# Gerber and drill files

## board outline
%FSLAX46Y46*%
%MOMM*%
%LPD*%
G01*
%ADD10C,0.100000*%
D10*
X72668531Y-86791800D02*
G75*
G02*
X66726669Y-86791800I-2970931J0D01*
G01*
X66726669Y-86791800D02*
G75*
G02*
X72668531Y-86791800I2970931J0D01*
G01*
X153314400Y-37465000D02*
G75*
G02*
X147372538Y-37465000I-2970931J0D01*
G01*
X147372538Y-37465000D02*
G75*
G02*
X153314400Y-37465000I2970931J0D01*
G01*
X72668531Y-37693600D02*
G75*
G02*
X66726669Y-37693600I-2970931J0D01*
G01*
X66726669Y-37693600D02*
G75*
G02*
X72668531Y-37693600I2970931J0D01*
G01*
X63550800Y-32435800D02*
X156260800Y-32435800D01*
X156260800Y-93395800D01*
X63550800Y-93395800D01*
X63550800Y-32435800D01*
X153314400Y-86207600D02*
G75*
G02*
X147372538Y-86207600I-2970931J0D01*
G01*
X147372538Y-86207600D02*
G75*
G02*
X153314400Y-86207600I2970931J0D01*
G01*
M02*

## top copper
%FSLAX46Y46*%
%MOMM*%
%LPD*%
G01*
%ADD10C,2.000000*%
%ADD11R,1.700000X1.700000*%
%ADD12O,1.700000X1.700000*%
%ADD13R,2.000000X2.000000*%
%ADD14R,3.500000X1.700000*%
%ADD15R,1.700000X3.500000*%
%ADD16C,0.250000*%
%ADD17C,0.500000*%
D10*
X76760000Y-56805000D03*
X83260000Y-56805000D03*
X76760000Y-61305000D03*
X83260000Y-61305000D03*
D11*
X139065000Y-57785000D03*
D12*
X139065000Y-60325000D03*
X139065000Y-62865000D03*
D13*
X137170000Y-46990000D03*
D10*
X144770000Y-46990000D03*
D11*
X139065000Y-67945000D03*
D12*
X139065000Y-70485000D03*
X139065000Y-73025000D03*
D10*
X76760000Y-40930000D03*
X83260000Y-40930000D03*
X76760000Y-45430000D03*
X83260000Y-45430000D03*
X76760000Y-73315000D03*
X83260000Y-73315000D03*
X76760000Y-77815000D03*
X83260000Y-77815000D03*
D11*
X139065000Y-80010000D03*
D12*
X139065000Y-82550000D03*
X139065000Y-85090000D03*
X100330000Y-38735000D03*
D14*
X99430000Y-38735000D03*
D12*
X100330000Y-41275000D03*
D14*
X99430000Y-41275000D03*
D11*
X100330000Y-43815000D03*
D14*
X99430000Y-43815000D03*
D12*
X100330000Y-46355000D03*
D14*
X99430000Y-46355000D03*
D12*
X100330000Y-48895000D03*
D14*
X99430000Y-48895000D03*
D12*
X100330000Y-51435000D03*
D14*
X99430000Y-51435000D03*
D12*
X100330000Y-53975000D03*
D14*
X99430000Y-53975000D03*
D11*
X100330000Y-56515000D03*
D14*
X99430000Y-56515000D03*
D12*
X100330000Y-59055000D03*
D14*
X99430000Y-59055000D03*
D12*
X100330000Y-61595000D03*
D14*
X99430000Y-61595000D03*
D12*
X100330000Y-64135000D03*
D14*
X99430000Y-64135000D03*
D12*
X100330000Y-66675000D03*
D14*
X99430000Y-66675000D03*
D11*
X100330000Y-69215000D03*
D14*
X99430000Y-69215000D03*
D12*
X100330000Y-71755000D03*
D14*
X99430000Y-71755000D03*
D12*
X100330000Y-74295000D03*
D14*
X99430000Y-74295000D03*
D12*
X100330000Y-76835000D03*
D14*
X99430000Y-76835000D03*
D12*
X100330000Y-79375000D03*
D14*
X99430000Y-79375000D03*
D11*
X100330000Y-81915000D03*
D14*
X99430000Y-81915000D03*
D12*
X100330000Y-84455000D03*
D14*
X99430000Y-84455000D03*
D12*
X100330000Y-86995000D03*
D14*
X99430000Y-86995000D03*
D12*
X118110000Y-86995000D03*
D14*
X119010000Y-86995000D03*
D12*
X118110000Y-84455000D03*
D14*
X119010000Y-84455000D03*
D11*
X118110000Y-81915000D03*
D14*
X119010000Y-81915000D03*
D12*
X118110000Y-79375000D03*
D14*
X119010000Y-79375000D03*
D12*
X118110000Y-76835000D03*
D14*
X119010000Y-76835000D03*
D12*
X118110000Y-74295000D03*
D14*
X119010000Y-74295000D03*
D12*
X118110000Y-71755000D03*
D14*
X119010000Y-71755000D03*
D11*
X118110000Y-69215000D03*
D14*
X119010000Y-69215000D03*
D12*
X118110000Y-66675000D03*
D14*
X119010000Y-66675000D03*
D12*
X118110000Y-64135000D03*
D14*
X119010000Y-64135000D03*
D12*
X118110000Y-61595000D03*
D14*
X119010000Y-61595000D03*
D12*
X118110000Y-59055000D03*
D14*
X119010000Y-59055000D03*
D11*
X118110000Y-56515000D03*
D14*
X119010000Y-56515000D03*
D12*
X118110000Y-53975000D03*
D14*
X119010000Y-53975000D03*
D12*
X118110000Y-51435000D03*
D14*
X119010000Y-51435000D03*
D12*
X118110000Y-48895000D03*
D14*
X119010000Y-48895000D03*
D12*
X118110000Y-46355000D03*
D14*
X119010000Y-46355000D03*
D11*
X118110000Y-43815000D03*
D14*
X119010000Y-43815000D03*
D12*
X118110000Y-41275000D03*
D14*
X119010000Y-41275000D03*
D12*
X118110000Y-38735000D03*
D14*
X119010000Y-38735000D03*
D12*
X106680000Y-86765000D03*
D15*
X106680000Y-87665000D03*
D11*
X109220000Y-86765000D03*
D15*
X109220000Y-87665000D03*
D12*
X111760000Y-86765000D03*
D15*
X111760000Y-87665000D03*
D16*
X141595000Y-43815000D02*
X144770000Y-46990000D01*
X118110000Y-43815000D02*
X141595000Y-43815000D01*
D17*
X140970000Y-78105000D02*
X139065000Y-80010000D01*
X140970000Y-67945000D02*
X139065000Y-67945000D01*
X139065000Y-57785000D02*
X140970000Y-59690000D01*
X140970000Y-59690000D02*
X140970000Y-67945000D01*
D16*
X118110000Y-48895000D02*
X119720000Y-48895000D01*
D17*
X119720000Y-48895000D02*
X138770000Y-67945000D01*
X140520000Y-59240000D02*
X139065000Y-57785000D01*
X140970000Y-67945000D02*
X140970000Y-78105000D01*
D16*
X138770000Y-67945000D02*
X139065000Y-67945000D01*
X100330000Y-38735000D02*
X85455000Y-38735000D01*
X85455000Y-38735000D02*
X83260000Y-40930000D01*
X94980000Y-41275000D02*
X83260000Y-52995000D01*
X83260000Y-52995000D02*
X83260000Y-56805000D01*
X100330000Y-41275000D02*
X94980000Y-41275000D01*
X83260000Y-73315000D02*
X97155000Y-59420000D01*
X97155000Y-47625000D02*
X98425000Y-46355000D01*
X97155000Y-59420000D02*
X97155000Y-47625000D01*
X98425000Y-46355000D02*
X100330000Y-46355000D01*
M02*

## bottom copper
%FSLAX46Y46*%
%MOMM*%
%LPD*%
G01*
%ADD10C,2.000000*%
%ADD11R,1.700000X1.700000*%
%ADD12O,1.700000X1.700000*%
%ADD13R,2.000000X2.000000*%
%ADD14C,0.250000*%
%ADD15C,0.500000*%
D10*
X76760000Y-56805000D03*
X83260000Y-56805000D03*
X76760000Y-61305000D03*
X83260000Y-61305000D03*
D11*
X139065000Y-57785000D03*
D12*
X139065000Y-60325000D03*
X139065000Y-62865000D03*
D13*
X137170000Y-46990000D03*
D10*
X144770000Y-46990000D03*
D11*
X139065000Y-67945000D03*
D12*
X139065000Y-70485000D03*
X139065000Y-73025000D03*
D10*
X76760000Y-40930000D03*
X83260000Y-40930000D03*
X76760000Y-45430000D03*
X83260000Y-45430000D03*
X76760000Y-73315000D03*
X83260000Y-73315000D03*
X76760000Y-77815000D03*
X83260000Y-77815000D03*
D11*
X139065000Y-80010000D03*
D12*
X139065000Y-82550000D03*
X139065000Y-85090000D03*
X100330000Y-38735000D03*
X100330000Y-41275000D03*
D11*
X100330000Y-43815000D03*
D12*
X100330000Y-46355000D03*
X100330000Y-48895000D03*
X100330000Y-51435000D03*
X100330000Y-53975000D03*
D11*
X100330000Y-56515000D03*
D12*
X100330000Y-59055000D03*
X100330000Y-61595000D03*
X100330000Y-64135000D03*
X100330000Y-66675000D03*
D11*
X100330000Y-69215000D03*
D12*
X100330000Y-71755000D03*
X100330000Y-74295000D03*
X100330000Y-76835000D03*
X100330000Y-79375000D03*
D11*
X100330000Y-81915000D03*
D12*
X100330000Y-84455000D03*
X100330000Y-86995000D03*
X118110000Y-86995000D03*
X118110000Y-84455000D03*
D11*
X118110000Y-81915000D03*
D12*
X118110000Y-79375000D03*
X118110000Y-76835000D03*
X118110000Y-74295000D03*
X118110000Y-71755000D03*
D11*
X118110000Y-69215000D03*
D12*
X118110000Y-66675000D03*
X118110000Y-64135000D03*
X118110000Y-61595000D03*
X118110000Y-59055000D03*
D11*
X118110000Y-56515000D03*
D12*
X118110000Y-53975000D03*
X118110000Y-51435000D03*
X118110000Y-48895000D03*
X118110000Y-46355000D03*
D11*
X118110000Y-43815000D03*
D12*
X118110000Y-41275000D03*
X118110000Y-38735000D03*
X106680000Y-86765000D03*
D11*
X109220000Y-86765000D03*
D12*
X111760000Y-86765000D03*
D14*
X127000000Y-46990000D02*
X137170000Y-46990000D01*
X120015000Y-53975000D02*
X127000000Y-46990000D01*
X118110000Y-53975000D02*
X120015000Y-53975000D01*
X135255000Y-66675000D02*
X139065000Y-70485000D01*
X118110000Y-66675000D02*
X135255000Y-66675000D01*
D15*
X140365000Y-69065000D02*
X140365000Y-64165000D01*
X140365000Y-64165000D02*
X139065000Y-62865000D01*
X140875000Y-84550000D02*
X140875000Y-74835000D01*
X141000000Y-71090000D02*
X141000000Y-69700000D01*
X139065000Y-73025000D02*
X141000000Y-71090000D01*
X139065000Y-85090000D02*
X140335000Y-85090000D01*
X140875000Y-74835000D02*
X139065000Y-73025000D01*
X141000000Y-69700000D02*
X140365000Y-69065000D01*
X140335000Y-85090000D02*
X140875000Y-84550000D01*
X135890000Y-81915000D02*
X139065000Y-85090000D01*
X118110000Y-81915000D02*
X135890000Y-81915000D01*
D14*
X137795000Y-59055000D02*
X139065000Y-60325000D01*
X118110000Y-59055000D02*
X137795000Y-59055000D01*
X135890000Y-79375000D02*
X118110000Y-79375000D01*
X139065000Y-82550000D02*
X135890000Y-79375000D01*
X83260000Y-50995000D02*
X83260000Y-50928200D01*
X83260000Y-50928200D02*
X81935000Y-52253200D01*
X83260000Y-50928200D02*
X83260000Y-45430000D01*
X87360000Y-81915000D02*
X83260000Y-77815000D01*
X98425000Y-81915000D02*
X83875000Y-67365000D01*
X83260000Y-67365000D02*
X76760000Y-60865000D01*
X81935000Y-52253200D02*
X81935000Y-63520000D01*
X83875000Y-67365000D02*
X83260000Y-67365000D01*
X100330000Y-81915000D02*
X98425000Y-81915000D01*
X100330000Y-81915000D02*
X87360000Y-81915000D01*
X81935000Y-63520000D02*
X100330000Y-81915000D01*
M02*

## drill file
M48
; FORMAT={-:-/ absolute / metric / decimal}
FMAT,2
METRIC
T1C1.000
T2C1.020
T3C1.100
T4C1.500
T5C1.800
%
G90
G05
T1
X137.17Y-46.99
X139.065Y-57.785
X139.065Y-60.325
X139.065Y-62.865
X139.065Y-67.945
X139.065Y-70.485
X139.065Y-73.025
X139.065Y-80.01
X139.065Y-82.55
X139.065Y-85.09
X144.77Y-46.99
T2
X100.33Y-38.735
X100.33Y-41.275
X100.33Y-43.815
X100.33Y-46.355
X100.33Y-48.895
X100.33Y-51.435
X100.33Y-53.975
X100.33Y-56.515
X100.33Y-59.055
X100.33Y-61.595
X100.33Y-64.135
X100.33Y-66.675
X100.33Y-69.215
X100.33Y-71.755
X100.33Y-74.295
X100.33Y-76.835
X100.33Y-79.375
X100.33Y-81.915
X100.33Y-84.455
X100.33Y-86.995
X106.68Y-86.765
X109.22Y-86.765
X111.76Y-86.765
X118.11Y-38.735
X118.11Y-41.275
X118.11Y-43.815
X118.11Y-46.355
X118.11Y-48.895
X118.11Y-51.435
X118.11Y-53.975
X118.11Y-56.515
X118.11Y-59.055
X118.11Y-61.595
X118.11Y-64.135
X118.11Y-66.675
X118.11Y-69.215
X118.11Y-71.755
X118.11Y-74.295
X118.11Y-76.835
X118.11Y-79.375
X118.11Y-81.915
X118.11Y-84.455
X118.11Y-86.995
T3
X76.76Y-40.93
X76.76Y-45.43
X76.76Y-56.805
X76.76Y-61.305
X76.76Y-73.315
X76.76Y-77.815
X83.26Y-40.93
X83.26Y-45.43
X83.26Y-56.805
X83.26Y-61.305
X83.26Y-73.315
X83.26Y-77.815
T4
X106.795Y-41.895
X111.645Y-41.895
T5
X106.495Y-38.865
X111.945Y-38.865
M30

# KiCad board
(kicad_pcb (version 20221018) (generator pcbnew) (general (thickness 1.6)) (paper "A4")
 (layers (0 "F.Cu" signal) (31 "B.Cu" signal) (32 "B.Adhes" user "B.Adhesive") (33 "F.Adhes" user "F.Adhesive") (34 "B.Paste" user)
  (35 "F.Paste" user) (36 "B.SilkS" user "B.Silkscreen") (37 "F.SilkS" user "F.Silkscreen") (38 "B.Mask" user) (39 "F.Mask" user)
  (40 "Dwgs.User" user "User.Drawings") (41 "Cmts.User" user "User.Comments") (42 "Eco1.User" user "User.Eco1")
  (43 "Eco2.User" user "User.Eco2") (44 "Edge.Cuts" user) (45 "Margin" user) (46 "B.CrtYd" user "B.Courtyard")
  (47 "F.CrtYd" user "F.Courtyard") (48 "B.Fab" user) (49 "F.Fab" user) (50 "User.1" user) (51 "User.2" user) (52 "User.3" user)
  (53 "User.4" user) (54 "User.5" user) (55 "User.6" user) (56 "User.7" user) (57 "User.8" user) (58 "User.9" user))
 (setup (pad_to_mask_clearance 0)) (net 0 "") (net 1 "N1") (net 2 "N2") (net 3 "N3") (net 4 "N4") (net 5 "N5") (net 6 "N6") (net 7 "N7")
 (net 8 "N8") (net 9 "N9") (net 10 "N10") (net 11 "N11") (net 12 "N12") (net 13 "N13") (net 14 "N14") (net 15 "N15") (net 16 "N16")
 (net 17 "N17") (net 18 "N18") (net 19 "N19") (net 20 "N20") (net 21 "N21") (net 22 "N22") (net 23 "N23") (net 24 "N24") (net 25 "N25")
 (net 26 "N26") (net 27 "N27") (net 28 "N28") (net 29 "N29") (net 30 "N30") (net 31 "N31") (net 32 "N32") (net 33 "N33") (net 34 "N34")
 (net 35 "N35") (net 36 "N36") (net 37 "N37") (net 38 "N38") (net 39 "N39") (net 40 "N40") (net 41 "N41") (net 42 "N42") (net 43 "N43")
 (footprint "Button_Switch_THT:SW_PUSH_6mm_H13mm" (layer "F.Cu") (at 76.76 56.805)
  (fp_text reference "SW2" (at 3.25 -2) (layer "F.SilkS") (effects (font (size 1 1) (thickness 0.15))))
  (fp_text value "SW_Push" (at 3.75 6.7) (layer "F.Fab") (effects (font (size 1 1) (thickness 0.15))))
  (pad "1" thru_hole circle (at 0 0 90) (size 2 2) (drill 1.1) (layers "*.Cu" "*.Mask") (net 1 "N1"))
  (pad "1" thru_hole circle (at 6.5 0 90) (size 2 2) (drill 1.1) (layers "*.Cu" "*.Mask") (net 1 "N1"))
  (pad "2" thru_hole circle (at 0 4.5 90) (size 2 2) (drill 1.1) (layers "*.Cu" "*.Mask") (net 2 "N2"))
  (pad "2" thru_hole circle (at 6.5 4.5 90) (size 2 2) (drill 1.1) (layers "*.Cu" "*.Mask") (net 2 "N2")))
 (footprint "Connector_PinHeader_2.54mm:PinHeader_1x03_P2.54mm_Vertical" (layer "F.Cu") (at 139.065 57.785)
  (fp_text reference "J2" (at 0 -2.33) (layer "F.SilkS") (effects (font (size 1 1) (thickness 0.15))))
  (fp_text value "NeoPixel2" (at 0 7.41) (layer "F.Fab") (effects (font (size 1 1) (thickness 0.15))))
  (pad "1" thru_hole rect (at 0 0) (size 1.7 1.7) (drill 1) (layers "*.Cu" "*.Mask") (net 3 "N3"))
  (pad "2" thru_hole oval (at 0 2.54) (size 1.7 1.7) (drill 1) (layers "*.Cu" "*.Mask") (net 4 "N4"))
  (pad "3" thru_hole oval (at 0 5.08) (size 1.7 1.7) (drill 1) (layers "*.Cu" "*.Mask") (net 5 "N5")))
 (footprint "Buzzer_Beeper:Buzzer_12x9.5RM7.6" (layer "F.Cu") (at 137.17 46.99)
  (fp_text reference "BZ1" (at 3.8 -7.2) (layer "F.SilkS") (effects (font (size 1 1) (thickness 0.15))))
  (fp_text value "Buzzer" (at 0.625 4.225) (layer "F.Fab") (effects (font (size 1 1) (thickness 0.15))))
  (pad "1" thru_hole rect (at 0 0) (size 2 2) (drill 1) (layers "*.Cu" "*.Mask") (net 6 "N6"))
  (pad "2" thru_hole circle (at 7.6 0) (size 2 2) (drill 1) (layers "*.Cu" "*.Mask") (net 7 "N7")))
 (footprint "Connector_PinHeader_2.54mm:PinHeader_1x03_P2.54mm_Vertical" (layer "F.Cu") (at 139.065 67.945)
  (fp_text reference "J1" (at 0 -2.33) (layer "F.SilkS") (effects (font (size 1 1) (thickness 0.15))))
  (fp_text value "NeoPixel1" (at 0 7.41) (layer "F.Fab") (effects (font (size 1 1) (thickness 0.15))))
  (pad "1" thru_hole rect (at 0 0) (size 1.7 1.7) (drill 1) (layers "*.Cu" "*.Mask") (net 3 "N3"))
  (pad "2" thru_hole oval (at 0 2.54) (size 1.7 1.7) (drill 1) (layers "*.Cu" "*.Mask") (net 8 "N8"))
  (pad "3" thru_hole oval (at 0 5.08) (size 1.7 1.7) (drill 1) (layers "*.Cu" "*.Mask") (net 5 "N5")))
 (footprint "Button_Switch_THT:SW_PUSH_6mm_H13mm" (layer "F.Cu") (at 76.76 40.93)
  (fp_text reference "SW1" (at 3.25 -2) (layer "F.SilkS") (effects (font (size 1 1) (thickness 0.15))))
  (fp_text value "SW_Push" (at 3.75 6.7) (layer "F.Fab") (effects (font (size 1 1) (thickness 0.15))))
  (pad "1" thru_hole circle (at 0 0 90) (size 2 2) (drill 1.1) (layers "*.Cu" "*.Mask") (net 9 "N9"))
  (pad "1" thru_hole circle (at 6.5 0 90) (size 2 2) (drill 1.1) (layers "*.Cu" "*.Mask") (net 9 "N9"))
  (pad "2" thru_hole circle (at 0 4.5 90) (size 2 2) (drill 1.1) (layers "*.Cu" "*.Mask") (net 2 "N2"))
  (pad "2" thru_hole circle (at 6.5 4.5 90) (size 2 2) (drill 1.1) (layers "*.Cu" "*.Mask") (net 2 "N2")))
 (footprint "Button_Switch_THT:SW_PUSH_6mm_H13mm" (layer "F.Cu") (at 76.76 73.315)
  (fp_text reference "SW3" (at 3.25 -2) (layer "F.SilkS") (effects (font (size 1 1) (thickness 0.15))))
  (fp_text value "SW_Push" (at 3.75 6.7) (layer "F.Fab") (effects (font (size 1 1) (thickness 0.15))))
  (pad "1" thru_hole circle (at 0 0 90) (size 2 2) (drill 1.1) (layers "*.Cu" "*.Mask") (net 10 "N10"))
  (pad "1" thru_hole circle (at 6.5 0 90) (size 2 2) (drill 1.1) (layers "*.Cu" "*.Mask") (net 10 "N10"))
  (pad "2" thru_hole circle (at 0 4.5 90) (size 2 2) (drill 1.1) (layers "*.Cu" "*.Mask") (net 2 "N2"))
  (pad "2" thru_hole circle (at 6.5 4.5 90) (size 2 2) (drill 1.1) (layers "*.Cu" "*.Mask") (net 2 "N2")))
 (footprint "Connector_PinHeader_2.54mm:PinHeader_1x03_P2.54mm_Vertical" (layer "F.Cu") (at 139.065 80.01)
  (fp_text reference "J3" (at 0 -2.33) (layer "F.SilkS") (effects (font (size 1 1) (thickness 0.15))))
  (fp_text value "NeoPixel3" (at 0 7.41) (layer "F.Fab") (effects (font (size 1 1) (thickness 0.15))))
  (pad "1" thru_hole rect (at 0 0) (size 1.7 1.7) (drill 1) (layers "*.Cu" "*.Mask") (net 3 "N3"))
  (pad "2" thru_hole oval (at 0 2.54) (size 1.7 1.7) (drill 1) (layers "*.Cu" "*.Mask") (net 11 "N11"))
  (pad "3" thru_hole oval (at 0 5.08) (size 1.7 1.7) (drill 1) (layers "*.Cu" "*.Mask") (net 5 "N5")))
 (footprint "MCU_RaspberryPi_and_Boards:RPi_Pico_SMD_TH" (layer "F.Cu") (at 109.22 62.865)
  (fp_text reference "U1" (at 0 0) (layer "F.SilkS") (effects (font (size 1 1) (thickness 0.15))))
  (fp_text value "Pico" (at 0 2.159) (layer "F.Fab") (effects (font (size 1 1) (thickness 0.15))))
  (pad "" np_thru_hole oval (at -2.725 -24) (size 1.8 1.8) (drill 1.8) (layers "*.Cu" "*.Mask"))
  (pad "" np_thru_hole oval (at -2.425 -20.97) (size 1.5 1.5) (drill 1.5) (layers "*.Cu" "*.Mask"))
  (pad "" np_thru_hole oval (at 2.425 -20.97) (size 1.5 1.5) (drill 1.5) (layers "*.Cu" "*.Mask"))
  (pad "" np_thru_hole oval (at 2.725 -24) (size 1.8 1.8) (drill 1.8) (layers "*.Cu" "*.Mask"))
  (pad "1" thru_hole oval (at -8.89 -24.13) (size 1.7 1.7) (drill 1.02) (layers "*.Cu" "*.Mask") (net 9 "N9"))
  (pad "1" smd rect (at -8.89 -24.13) (size 3.5 1.7) (drill (offset -0.9 0)) (layers "F.Cu" "F.Mask") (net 9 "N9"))
  (pad "2" thru_hole oval (at -8.89 -21.59) (size 1.7 1.7) (drill 1.02) (layers "*.Cu" "*.Mask") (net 1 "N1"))
  (pad "2" smd rect (at -8.89 -21.59) (size 3.5 1.7) (drill (offset -0.9 0)) (layers "F.Cu" "F.Mask") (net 1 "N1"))
  (pad "3" thru_hole rect (at -8.89 -19.05) (size 1.7 1.7) (drill 1.02) (layers "*.Cu" "*.Mask") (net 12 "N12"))
  (pad "3" smd rect (at -8.89 -19.05) (size 3.5 1.7) (drill (offset -0.9 0)) (layers "F.Cu" "F.Mask") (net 12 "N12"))
  (pad "4" thru_hole oval (at -8.89 -16.51) (size 1.7 1.7) (drill 1.02) (layers "*.Cu" "*.Mask") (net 10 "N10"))
  (pad "4" smd rect (at -8.89 -16.51) (size 3.5 1.7) (drill (offset -0.9 0)) (layers "F.Cu" "F.Mask") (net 10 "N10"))
  (pad "5" thru_hole oval (at -8.89 -13.97) (size 1.7 1.7) (drill 1.02) (layers "*.Cu" "*.Mask") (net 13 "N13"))
  (pad "5" smd rect (at -8.89 -13.97) (size 3.5 1.7) (drill (offset -0.9 0)) (layers "F.Cu" "F.Mask") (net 13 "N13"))
  (pad "6" thru_hole oval (at -8.89 -11.43) (size 1.7 1.7) (drill 1.02) (layers "*.Cu" "*.Mask") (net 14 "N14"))
  (pad "6" smd rect (at -8.89 -11.43) (size 3.5 1.7) (drill (offset -0.9 0)) (layers "F.Cu" "F.Mask") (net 14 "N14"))
  (pad "7" thru_hole oval (at -8.89 -8.89) (size 1.7 1.7) (drill 1.02) (layers "*.Cu" "*.Mask") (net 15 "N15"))
  (pad "7" smd rect (at -8.89 -8.89) (size 3.5 1.7) (drill (offset -0.9 0)) (layers "F.Cu" "F.Mask") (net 15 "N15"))
  (pad "8" thru_hole rect (at -8.89 -6.35) (size 1.7 1.7) (drill 1.02) (layers "*.Cu" "*.Mask") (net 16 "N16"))
  (pad "8" smd rect (at -8.89 -6.35) (size 3.5 1.7) (drill (offset -0.9 0)) (layers "F.Cu" "F.Mask") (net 16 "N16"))
  (pad "9" thru_hole oval (at -8.89 -3.81) (size 1.7 1.7) (drill 1.02) (layers "*.Cu" "*.Mask") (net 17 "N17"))
  (pad "9" smd rect (at -8.89 -3.81) (size 3.5 1.7) (drill (offset -0.9 0)) (layers "F.Cu" "F.Mask") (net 17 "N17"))
  (pad "10" thru_hole oval (at -8.89 -1.27) (size 1.7 1.7) (drill 1.02) (layers "*.Cu" "*.Mask") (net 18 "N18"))
  (pad "10" smd rect (at -8.89 -1.27) (size 3.5 1.7) (drill (offset -0.9 0)) (layers "F.Cu" "F.Mask") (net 18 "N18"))
  (pad "11" thru_hole oval (at -8.89 1.27) (size 1.7 1.7) (drill 1.02) (layers "*.Cu" "*.Mask") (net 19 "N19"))
  (pad "11" smd rect (at -8.89 1.27) (size 3.5 1.7) (drill (offset -0.9 0)) (layers "F.Cu" "F.Mask") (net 19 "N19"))
  (pad "12" thru_hole oval (at -8.89 3.81) (size 1.7 1.7) (drill 1.02) (layers "*.Cu" "*.Mask") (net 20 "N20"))
  (pad "12" smd rect (at -8.89 3.81) (size 3.5 1.7) (drill (offset -0.9 0)) (layers "F.Cu" "F.Mask") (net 20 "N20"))
  (pad "13" thru_hole rect (at -8.89 6.35) (size 1.7 1.7) (drill 1.02) (layers "*.Cu" "*.Mask") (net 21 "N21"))
  (pad "13" smd rect (at -8.89 6.35) (size 3.5 1.7) (drill (offset -0.9 0)) (layers "F.Cu" "F.Mask") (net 21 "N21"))
  (pad "14" thru_hole oval (at -8.89 8.89) (size 1.7 1.7) (drill 1.02) (layers "*.Cu" "*.Mask") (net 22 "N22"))
  (pad "14" smd rect (at -8.89 8.89) (size 3.5 1.7) (drill (offset -0.9 0)) (layers "F.Cu" "F.Mask") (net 22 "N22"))
  (pad "15" thru_hole oval (at -8.89 11.43) (size 1.7 1.7) (drill 1.02) (layers "*.Cu" "*.Mask") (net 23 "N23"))
  (pad "15" smd rect (at -8.89 11.43) (size 3.5 1.7) (drill (offset -0.9 0)) (layers "F.Cu" "F.Mask") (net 23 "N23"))
  (pad "16" thru_hole oval (at -8.89 13.97) (size 1.7 1.7) (drill 1.02) (layers "*.Cu" "*.Mask") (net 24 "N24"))
  (pad "16" smd rect (at -8.89 13.97) (size 3.5 1.7) (drill (offset -0.9 0)) (layers "F.Cu" "F.Mask") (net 24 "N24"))
  (pad "17" thru_hole oval (at -8.89 16.51) (size 1.7 1.7) (drill 1.02) (layers "*.Cu" "*.Mask") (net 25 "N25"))
  (pad "17" smd rect (at -8.89 16.51) (size 3.5 1.7) (drill (offset -0.9 0)) (layers "F.Cu" "F.Mask") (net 25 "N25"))
  (pad "18" thru_hole rect (at -8.89 19.05) (size 1.7 1.7) (drill 1.02) (layers "*.Cu" "*.Mask") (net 2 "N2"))
  (pad "18" smd rect (at -8.89 19.05) (size 3.5 1.7) (drill (offset -0.9 0)) (layers "F.Cu" "F.Mask") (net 2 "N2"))
  (pad "19" thru_hole oval (at -8.89 21.59) (size 1.7 1.7) (drill 1.02) (layers "*.Cu" "*.Mask") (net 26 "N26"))
  (pad "19" smd rect (at -8.89 21.59) (size 3.5 1.7) (drill (offset -0.9 0)) (layers "F.Cu" "F.Mask") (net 26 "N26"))
  (pad "20" thru_hole oval (at -8.89 24.13) (size 1.7 1.7) (drill 1.02) (layers "*.Cu" "*.Mask") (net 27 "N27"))
  (pad "20" smd rect (at -8.89 24.13) (size 3.5 1.7) (drill (offset -0.9 0)) (layers "F.Cu" "F.Mask") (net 27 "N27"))
  (pad "21" thru_hole oval (at 8.89 24.13) (size 1.7 1.7) (drill 1.02) (layers "*.Cu" "*.Mask") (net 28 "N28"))
  (pad "21" smd rect (at 8.89 24.13) (size 3.5 1.7) (drill (offset 0.9 0)) (layers "F.Cu" "F.Mask") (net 28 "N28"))
  (pad "22" thru_hole oval (at 8.89 21.59) (size 1.7 1.7) (drill 1.02) (layers "*.Cu" "*.Mask") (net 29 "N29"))
  (pad "22" smd rect (at 8.89 21.59) (size 3.5 1.7) (drill (offset 0.9 0)) (layers "F.Cu" "F.Mask") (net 29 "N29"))
  (pad "23" thru_hole rect (at 8.89 19.05) (size 1.7 1.7) (drill 1.02) (layers "*.Cu" "*.Mask") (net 5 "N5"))
  (pad "23" smd rect (at 8.89 19.05) (size 3.5 1.7) (drill (offset 0.9 0)) (layers "F.Cu" "F.Mask") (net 5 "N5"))
  (pad "24" thru_hole oval (at 8.89 16.51) (size 1.7 1.7) (drill 1.02) (layers "*.Cu" "*.Mask") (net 11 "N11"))
  (pad "24" smd rect (at 8.89 16.51) (size 3.5 1.7) (drill (offset 0.9 0)) (layers "F.Cu" "F.Mask") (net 11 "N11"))
  (pad "25" thru_hole oval (at 8.89 13.97) (size 1.7 1.7) (drill 1.02) (layers "*.Cu" "*.Mask") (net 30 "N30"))
  (pad "25" smd rect (at 8.89 13.97) (size 3.5 1.7) (drill (offset 0.9 0)) (layers "F.Cu" "F.Mask") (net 30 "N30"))
  (pad "26" thru_hole oval (at 8.89 11.43) (size 1.7 1.7) (drill 1.02) (layers "*.Cu" "*.Mask") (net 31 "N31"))
  (pad "26" smd rect (at 8.89 11.43) (size 3.5 1.7) (drill (offset 0.9 0)) (layers "F.Cu" "F.Mask") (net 31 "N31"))
  (pad "27" thru_hole oval (at 8.89 8.89) (size 1.7 1.7) (drill 1.02) (layers "*.Cu" "*.Mask") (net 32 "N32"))
  (pad "27" smd rect (at 8.89 8.89) (size 3.5 1.7) (drill (offset 0.9 0)) (layers "F.Cu" "F.Mask") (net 32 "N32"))
  (pad "28" thru_hole rect (at 8.89 6.35) (size 1.7 1.7) (drill 1.02) (layers "*.Cu" "*.Mask") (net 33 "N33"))
  (pad "28" smd rect (at 8.89 6.35) (size 3.5 1.7) (drill (offset 0.9 0)) (layers "F.Cu" "F.Mask") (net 33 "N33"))
  (pad "29" thru_hole oval (at 8.89 3.81) (size 1.7 1.7) (drill 1.02) (layers "*.Cu" "*.Mask") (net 8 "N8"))
  (pad "29" smd rect (at 8.89 3.81) (size 3.5 1.7) (drill (offset 0.9 0)) (layers "F.Cu" "F.Mask") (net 8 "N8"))
  (pad "30" thru_hole oval (at 8.89 1.27) (size 1.7 1.7) (drill 1.02) (layers "*.Cu" "*.Mask") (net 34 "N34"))
  (pad "30" smd rect (at 8.89 1.27) (size 3.5 1.7) (drill (offset 0.9 0)) (layers "F.Cu" "F.Mask") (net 34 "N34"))
  (pad "31" thru_hole oval (at 8.89 -1.27) (size 1.7 1.7) (drill 1.02) (layers "*.Cu" "*.Mask") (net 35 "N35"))
  (pad "31" smd rect (at 8.89 -1.27) (size 3.5 1.7) (drill (offset 0.9 0)) (layers "F.Cu" "F.Mask") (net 35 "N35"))
  (pad "32" thru_hole oval (at 8.89 -3.81) (size 1.7 1.7) (drill 1.02) (layers "*.Cu" "*.Mask") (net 4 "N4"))
  (pad "32" smd rect (at 8.89 -3.81) (size 3.5 1.7) (drill (offset 0.9 0)) (layers "F.Cu" "F.Mask") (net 4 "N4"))
  (pad "33" thru_hole rect (at 8.89 -6.35) (size 1.7 1.7) (drill 1.02) (layers "*.Cu" "*.Mask") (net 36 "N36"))
  (pad "33" smd rect (at 8.89 -6.35) (size 3.5 1.7) (drill (offset 0.9 0)) (layers "F.Cu" "F.Mask") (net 36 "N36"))
  (pad "34" thru_hole oval (at 8.89 -8.89) (size 1.7 1.7) (drill 1.02) (layers "*.Cu" "*.Mask") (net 6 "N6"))
  (pad "34" smd rect (at 8.89 -8.89) (size 3.5 1.7) (drill (offset 0.9 0)) (layers "F.Cu" "F.Mask") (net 6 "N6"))
  (pad "35" thru_hole oval (at 8.89 -11.43) (size 1.7 1.7) (drill 1.02) (layers "*.Cu" "*.Mask") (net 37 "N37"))
  (pad "35" smd rect (at 8.89 -11.43) (size 3.5 1.7) (drill (offset 0.9 0)) (layers "F.Cu" "F.Mask") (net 37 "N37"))
  (pad "36" thru_hole oval (at 8.89 -13.97) (size 1.7 1.7) (drill 1.02) (layers "*.Cu" "*.Mask") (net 3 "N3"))
  (pad "36" smd rect (at 8.89 -13.97) (size 3.5 1.7) (drill (offset 0.9 0)) (layers "F.Cu" "F.Mask") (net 3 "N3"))
  (pad "37" thru_hole oval (at 8.89 -16.51) (size 1.7 1.7) (drill 1.02) (layers "*.Cu" "*.Mask") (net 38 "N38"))
  (pad "37" smd rect (at 8.89 -16.51) (size 3.5 1.7) (drill (offset 0.9 0)) (layers "F.Cu" "F.Mask") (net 38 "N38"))
  (pad "38" thru_hole rect (at 8.89 -19.05) (size 1.7 1.7) (drill 1.02) (layers "*.Cu" "*.Mask") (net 7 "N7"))
  (pad "38" smd rect (at 8.89 -19.05) (size 3.5 1.7) (drill (offset 0.9 0)) (layers "F.Cu" "F.Mask") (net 7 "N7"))
  (pad "39" thru_hole oval (at 8.89 -21.59) (size 1.7 1.7) (drill 1.02) (layers "*.Cu" "*.Mask") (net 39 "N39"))
  (pad "39" smd rect (at 8.89 -21.59) (size 3.5 1.7) (drill (offset 0.9 0)) (layers "F.Cu" "F.Mask") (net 39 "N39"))
  (pad "40" thru_hole oval (at 8.89 -24.13) (size 1.7 1.7) (drill 1.02) (layers "*.Cu" "*.Mask") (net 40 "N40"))
  (pad "40" smd rect (at 8.89 -24.13) (size 3.5 1.7) (drill (offset 0.9 0)) (layers "F.Cu" "F.Mask") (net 40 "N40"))
  (pad "41" thru_hole oval (at -2.54 23.9) (size 1.7 1.7) (drill 1.02) (layers "*.Cu" "*.Mask") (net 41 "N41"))
  (pad "41" smd rect (at -2.54 23.9 90) (size 3.5 1.7) (drill (offset -0.9 0)) (layers "F.Cu" "F.Mask") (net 41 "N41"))
  (pad "42" thru_hole rect (at 0 23.9) (size 1.7 1.7) (drill 1.02) (layers "*.Cu" "*.Mask") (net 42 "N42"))
  (pad "42" smd rect (at 0 23.9 90) (size 3.5 1.7) (drill (offset -0.9 0)) (layers "F.Cu" "F.Mask") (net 42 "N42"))
  (pad "43" thru_hole oval (at 2.54 23.9) (size 1.7 1.7) (drill 1.02) (layers "*.Cu" "*.Mask") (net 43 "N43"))
  (pad "43" smd rect (at 2.54 23.9 90) (size 3.5 1.7) (drill (offset -0.9 0)) (layers "F.Cu" "F.Mask") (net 43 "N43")))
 (gr_circle (center 69.6976 86.7918) (end 70.0786 89.7382) (stroke (width 0.1) (type solid)) (fill none) (layer "Edge.Cuts"))
 (gr_circle (center 150.343469 37.465) (end 150.724469 40.4114) (stroke (width 0.1) (type solid)) (fill none) (layer "Edge.Cuts"))
 (gr_circle (center 69.6976 37.6936) (end 70.0786 40.64) (stroke (width 0.1) (type solid)) (fill none) (layer "Edge.Cuts"))
 (gr_rect (start 63.5508 32.4358) (end 156.2608 93.3958) (stroke (width 0.1) (type solid)) (fill none) (layer "Edge.Cuts"))
 (gr_circle (center 150.343469 86.2076) (end 150.724469 89.154) (stroke (width 0.1) (type solid)) (fill none) (layer "Edge.Cuts"))
 (segment (start 127 46.99) (end 137.17 46.99) (width 0.25) (layer "B.Cu") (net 6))
 (segment (start 120.015 53.975) (end 127 46.99) (width 0.25) (layer "B.Cu") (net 6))
 (segment (start 118.11 53.975) (end 120.015 53.975) (width 0.25) (layer "B.Cu") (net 6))
 (segment (start 141.595 43.815) (end 144.77 46.99) (width 0.25) (layer "F.Cu") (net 7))
 (segment (start 118.11 43.815) (end 141.595 43.815) (width 0.25) (layer "F.Cu") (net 7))
 (segment (start 140.97 78.105) (end 139.065 80.01) (width 0.5) (layer "F.Cu") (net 3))
 (segment (start 140.97 67.945) (end 139.065 67.945) (width 0.5) (layer "F.Cu") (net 3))
 (segment (start 139.065 57.785) (end 140.97 59.69) (width 0.5) (layer "F.Cu") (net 3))
 (segment (start 140.97 59.69) (end 140.97 67.945) (width 0.5) (layer "F.Cu") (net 3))
 (segment (start 118.11 48.895) (end 119.72 48.895) (width 0.25) (layer "F.Cu") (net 3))
 (segment (start 119.72 48.895) (end 138.77 67.945) (width 0.5) (layer "F.Cu") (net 3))
 (segment (start 140.52 59.24) (end 139.065 57.785) (width 0.5) (layer "F.Cu") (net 3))
 (segment (start 140.97 67.945) (end 140.97 78.105) (width 0.5) (layer "F.Cu") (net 3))
 (segment (start 138.77 67.945) (end 139.065 67.945) (width 0.25) (layer "F.Cu") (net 3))
 (segment (start 135.255 66.675) (end 139.065 70.485) (width 0.25) (layer "B.Cu") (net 8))
 (segment (start 118.11 66.675) (end 135.255 66.675) (width 0.25) (layer "B.Cu") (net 8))
 (segment (start 140.365 69.065) (end 140.365 64.165) (width 0.5) (layer "B.Cu") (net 5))
 (segment (start 140.365 64.165) (end 139.065 62.865) (width 0.5) (layer "B.Cu") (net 5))
 (segment (start 140.875 84.55) (end 140.875 74.835) (width 0.5) (layer "B.Cu") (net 5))
 (segment (start 141 71.09) (end 141 69.7) (width 0.5) (layer "B.Cu") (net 5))
 (segment (start 139.065 73.025) (end 141 71.09) (width 0.5) (layer "B.Cu") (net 5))
 (segment (start 139.065 85.09) (end 140.335 85.09) (width 0.5) (layer "B.Cu") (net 5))
 (segment (start 140.875 74.835) (end 139.065 73.025) (width 0.5) (layer "B.Cu") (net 5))
 (segment (start 141 69.7) (end 140.365 69.065) (width 0.5) (layer "B.Cu") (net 5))
 (segment (start 140.335 85.09) (end 140.875 84.55) (width 0.5) (layer "B.Cu") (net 5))
 (segment (start 135.89 81.915) (end 139.065 85.09) (width 0.5) (layer "B.Cu") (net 5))
 (segment (start 118.11 81.915) (end 135.89 81.915) (width 0.5) (layer "B.Cu") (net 5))
 (segment (start 137.795 59.055) (end 139.065 60.325) (width 0.25) (layer "B.Cu") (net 4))
 (segment (start 118.11 59.055) (end 137.795 59.055) (width 0.25) (layer "B.Cu") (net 4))
 (segment (start 135.89 79.375) (end 118.11 79.375) (width 0.25) (layer "B.Cu") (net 11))
 (segment (start 139.065 82.55) (end 135.89 79.375) (width 0.25) (layer "B.Cu") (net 11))
 (segment (start 100.33 38.735) (end 85.455 38.735) (width 0.25) (layer "F.Cu") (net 9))
 (segment (start 85.455 38.735) (end 83.26 40.93) (width 0.25) (layer "F.Cu") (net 9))
 (segment (start 83.26 50.995) (end 83.26 50.9282) (width 0.25) (layer "B.Cu") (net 2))
 (segment (start 83.26 50.9282) (end 81.935 52.2532) (width 0.25) (layer "B.Cu") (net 2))
 (segment (start 83.26 50.9282) (end 83.26 45.43) (width 0.25) (layer "B.Cu") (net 2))
 (segment (start 87.36 81.915) (end 83.26 77.815) (width 0.25) (layer "B.Cu") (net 2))
 (segment (start 98.425 81.915) (end 83.875 67.365) (width 0.25) (layer "B.Cu") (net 2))
 (segment (start 83.26 67.365) (end 76.76 60.865) (width 0.25) (layer "B.Cu") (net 2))
 (segment (start 81.935 52.2532) (end 81.935 63.52) (width 0.25) (layer "B.Cu") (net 2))
 (segment (start 83.875 67.365) (end 83.26 67.365) (width 0.25) (layer "B.Cu") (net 2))
 (segment (start 100.33 81.915) (end 98.425 81.915) (width 0.25) (layer "B.Cu") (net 2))
 (segment (start 100.33 81.915) (end 87.36 81.915) (width 0.25) (layer "B.Cu") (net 2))
 (segment (start 81.935 63.52) (end 100.33 81.915) (width 0.25) (layer "B.Cu") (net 2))
 (segment (start 94.98 41.275) (end 83.26 52.995) (width 0.25) (layer "F.Cu") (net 1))
 (segment (start 83.26 52.995) (end 83.26 56.805) (width 0.25) (layer "F.Cu") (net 1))
 (segment (start 100.33 41.275) (end 94.98 41.275) (width 0.25) (layer "F.Cu") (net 1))
 (segment (start 83.26 73.315) (end 97.155 59.42) (width 0.25) (layer "F.Cu") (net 10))
 (segment (start 97.155 47.625) (end 98.425 46.355) (width 0.25) (layer "F.Cu") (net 10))
 (segment (start 97.155 59.42) (end 97.155 47.625) (width 0.25) (layer "F.Cu") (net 10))
 (segment (start 98.425 46.355) (end 100.33 46.355) (width 0.25) (layer "F.Cu") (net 10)))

